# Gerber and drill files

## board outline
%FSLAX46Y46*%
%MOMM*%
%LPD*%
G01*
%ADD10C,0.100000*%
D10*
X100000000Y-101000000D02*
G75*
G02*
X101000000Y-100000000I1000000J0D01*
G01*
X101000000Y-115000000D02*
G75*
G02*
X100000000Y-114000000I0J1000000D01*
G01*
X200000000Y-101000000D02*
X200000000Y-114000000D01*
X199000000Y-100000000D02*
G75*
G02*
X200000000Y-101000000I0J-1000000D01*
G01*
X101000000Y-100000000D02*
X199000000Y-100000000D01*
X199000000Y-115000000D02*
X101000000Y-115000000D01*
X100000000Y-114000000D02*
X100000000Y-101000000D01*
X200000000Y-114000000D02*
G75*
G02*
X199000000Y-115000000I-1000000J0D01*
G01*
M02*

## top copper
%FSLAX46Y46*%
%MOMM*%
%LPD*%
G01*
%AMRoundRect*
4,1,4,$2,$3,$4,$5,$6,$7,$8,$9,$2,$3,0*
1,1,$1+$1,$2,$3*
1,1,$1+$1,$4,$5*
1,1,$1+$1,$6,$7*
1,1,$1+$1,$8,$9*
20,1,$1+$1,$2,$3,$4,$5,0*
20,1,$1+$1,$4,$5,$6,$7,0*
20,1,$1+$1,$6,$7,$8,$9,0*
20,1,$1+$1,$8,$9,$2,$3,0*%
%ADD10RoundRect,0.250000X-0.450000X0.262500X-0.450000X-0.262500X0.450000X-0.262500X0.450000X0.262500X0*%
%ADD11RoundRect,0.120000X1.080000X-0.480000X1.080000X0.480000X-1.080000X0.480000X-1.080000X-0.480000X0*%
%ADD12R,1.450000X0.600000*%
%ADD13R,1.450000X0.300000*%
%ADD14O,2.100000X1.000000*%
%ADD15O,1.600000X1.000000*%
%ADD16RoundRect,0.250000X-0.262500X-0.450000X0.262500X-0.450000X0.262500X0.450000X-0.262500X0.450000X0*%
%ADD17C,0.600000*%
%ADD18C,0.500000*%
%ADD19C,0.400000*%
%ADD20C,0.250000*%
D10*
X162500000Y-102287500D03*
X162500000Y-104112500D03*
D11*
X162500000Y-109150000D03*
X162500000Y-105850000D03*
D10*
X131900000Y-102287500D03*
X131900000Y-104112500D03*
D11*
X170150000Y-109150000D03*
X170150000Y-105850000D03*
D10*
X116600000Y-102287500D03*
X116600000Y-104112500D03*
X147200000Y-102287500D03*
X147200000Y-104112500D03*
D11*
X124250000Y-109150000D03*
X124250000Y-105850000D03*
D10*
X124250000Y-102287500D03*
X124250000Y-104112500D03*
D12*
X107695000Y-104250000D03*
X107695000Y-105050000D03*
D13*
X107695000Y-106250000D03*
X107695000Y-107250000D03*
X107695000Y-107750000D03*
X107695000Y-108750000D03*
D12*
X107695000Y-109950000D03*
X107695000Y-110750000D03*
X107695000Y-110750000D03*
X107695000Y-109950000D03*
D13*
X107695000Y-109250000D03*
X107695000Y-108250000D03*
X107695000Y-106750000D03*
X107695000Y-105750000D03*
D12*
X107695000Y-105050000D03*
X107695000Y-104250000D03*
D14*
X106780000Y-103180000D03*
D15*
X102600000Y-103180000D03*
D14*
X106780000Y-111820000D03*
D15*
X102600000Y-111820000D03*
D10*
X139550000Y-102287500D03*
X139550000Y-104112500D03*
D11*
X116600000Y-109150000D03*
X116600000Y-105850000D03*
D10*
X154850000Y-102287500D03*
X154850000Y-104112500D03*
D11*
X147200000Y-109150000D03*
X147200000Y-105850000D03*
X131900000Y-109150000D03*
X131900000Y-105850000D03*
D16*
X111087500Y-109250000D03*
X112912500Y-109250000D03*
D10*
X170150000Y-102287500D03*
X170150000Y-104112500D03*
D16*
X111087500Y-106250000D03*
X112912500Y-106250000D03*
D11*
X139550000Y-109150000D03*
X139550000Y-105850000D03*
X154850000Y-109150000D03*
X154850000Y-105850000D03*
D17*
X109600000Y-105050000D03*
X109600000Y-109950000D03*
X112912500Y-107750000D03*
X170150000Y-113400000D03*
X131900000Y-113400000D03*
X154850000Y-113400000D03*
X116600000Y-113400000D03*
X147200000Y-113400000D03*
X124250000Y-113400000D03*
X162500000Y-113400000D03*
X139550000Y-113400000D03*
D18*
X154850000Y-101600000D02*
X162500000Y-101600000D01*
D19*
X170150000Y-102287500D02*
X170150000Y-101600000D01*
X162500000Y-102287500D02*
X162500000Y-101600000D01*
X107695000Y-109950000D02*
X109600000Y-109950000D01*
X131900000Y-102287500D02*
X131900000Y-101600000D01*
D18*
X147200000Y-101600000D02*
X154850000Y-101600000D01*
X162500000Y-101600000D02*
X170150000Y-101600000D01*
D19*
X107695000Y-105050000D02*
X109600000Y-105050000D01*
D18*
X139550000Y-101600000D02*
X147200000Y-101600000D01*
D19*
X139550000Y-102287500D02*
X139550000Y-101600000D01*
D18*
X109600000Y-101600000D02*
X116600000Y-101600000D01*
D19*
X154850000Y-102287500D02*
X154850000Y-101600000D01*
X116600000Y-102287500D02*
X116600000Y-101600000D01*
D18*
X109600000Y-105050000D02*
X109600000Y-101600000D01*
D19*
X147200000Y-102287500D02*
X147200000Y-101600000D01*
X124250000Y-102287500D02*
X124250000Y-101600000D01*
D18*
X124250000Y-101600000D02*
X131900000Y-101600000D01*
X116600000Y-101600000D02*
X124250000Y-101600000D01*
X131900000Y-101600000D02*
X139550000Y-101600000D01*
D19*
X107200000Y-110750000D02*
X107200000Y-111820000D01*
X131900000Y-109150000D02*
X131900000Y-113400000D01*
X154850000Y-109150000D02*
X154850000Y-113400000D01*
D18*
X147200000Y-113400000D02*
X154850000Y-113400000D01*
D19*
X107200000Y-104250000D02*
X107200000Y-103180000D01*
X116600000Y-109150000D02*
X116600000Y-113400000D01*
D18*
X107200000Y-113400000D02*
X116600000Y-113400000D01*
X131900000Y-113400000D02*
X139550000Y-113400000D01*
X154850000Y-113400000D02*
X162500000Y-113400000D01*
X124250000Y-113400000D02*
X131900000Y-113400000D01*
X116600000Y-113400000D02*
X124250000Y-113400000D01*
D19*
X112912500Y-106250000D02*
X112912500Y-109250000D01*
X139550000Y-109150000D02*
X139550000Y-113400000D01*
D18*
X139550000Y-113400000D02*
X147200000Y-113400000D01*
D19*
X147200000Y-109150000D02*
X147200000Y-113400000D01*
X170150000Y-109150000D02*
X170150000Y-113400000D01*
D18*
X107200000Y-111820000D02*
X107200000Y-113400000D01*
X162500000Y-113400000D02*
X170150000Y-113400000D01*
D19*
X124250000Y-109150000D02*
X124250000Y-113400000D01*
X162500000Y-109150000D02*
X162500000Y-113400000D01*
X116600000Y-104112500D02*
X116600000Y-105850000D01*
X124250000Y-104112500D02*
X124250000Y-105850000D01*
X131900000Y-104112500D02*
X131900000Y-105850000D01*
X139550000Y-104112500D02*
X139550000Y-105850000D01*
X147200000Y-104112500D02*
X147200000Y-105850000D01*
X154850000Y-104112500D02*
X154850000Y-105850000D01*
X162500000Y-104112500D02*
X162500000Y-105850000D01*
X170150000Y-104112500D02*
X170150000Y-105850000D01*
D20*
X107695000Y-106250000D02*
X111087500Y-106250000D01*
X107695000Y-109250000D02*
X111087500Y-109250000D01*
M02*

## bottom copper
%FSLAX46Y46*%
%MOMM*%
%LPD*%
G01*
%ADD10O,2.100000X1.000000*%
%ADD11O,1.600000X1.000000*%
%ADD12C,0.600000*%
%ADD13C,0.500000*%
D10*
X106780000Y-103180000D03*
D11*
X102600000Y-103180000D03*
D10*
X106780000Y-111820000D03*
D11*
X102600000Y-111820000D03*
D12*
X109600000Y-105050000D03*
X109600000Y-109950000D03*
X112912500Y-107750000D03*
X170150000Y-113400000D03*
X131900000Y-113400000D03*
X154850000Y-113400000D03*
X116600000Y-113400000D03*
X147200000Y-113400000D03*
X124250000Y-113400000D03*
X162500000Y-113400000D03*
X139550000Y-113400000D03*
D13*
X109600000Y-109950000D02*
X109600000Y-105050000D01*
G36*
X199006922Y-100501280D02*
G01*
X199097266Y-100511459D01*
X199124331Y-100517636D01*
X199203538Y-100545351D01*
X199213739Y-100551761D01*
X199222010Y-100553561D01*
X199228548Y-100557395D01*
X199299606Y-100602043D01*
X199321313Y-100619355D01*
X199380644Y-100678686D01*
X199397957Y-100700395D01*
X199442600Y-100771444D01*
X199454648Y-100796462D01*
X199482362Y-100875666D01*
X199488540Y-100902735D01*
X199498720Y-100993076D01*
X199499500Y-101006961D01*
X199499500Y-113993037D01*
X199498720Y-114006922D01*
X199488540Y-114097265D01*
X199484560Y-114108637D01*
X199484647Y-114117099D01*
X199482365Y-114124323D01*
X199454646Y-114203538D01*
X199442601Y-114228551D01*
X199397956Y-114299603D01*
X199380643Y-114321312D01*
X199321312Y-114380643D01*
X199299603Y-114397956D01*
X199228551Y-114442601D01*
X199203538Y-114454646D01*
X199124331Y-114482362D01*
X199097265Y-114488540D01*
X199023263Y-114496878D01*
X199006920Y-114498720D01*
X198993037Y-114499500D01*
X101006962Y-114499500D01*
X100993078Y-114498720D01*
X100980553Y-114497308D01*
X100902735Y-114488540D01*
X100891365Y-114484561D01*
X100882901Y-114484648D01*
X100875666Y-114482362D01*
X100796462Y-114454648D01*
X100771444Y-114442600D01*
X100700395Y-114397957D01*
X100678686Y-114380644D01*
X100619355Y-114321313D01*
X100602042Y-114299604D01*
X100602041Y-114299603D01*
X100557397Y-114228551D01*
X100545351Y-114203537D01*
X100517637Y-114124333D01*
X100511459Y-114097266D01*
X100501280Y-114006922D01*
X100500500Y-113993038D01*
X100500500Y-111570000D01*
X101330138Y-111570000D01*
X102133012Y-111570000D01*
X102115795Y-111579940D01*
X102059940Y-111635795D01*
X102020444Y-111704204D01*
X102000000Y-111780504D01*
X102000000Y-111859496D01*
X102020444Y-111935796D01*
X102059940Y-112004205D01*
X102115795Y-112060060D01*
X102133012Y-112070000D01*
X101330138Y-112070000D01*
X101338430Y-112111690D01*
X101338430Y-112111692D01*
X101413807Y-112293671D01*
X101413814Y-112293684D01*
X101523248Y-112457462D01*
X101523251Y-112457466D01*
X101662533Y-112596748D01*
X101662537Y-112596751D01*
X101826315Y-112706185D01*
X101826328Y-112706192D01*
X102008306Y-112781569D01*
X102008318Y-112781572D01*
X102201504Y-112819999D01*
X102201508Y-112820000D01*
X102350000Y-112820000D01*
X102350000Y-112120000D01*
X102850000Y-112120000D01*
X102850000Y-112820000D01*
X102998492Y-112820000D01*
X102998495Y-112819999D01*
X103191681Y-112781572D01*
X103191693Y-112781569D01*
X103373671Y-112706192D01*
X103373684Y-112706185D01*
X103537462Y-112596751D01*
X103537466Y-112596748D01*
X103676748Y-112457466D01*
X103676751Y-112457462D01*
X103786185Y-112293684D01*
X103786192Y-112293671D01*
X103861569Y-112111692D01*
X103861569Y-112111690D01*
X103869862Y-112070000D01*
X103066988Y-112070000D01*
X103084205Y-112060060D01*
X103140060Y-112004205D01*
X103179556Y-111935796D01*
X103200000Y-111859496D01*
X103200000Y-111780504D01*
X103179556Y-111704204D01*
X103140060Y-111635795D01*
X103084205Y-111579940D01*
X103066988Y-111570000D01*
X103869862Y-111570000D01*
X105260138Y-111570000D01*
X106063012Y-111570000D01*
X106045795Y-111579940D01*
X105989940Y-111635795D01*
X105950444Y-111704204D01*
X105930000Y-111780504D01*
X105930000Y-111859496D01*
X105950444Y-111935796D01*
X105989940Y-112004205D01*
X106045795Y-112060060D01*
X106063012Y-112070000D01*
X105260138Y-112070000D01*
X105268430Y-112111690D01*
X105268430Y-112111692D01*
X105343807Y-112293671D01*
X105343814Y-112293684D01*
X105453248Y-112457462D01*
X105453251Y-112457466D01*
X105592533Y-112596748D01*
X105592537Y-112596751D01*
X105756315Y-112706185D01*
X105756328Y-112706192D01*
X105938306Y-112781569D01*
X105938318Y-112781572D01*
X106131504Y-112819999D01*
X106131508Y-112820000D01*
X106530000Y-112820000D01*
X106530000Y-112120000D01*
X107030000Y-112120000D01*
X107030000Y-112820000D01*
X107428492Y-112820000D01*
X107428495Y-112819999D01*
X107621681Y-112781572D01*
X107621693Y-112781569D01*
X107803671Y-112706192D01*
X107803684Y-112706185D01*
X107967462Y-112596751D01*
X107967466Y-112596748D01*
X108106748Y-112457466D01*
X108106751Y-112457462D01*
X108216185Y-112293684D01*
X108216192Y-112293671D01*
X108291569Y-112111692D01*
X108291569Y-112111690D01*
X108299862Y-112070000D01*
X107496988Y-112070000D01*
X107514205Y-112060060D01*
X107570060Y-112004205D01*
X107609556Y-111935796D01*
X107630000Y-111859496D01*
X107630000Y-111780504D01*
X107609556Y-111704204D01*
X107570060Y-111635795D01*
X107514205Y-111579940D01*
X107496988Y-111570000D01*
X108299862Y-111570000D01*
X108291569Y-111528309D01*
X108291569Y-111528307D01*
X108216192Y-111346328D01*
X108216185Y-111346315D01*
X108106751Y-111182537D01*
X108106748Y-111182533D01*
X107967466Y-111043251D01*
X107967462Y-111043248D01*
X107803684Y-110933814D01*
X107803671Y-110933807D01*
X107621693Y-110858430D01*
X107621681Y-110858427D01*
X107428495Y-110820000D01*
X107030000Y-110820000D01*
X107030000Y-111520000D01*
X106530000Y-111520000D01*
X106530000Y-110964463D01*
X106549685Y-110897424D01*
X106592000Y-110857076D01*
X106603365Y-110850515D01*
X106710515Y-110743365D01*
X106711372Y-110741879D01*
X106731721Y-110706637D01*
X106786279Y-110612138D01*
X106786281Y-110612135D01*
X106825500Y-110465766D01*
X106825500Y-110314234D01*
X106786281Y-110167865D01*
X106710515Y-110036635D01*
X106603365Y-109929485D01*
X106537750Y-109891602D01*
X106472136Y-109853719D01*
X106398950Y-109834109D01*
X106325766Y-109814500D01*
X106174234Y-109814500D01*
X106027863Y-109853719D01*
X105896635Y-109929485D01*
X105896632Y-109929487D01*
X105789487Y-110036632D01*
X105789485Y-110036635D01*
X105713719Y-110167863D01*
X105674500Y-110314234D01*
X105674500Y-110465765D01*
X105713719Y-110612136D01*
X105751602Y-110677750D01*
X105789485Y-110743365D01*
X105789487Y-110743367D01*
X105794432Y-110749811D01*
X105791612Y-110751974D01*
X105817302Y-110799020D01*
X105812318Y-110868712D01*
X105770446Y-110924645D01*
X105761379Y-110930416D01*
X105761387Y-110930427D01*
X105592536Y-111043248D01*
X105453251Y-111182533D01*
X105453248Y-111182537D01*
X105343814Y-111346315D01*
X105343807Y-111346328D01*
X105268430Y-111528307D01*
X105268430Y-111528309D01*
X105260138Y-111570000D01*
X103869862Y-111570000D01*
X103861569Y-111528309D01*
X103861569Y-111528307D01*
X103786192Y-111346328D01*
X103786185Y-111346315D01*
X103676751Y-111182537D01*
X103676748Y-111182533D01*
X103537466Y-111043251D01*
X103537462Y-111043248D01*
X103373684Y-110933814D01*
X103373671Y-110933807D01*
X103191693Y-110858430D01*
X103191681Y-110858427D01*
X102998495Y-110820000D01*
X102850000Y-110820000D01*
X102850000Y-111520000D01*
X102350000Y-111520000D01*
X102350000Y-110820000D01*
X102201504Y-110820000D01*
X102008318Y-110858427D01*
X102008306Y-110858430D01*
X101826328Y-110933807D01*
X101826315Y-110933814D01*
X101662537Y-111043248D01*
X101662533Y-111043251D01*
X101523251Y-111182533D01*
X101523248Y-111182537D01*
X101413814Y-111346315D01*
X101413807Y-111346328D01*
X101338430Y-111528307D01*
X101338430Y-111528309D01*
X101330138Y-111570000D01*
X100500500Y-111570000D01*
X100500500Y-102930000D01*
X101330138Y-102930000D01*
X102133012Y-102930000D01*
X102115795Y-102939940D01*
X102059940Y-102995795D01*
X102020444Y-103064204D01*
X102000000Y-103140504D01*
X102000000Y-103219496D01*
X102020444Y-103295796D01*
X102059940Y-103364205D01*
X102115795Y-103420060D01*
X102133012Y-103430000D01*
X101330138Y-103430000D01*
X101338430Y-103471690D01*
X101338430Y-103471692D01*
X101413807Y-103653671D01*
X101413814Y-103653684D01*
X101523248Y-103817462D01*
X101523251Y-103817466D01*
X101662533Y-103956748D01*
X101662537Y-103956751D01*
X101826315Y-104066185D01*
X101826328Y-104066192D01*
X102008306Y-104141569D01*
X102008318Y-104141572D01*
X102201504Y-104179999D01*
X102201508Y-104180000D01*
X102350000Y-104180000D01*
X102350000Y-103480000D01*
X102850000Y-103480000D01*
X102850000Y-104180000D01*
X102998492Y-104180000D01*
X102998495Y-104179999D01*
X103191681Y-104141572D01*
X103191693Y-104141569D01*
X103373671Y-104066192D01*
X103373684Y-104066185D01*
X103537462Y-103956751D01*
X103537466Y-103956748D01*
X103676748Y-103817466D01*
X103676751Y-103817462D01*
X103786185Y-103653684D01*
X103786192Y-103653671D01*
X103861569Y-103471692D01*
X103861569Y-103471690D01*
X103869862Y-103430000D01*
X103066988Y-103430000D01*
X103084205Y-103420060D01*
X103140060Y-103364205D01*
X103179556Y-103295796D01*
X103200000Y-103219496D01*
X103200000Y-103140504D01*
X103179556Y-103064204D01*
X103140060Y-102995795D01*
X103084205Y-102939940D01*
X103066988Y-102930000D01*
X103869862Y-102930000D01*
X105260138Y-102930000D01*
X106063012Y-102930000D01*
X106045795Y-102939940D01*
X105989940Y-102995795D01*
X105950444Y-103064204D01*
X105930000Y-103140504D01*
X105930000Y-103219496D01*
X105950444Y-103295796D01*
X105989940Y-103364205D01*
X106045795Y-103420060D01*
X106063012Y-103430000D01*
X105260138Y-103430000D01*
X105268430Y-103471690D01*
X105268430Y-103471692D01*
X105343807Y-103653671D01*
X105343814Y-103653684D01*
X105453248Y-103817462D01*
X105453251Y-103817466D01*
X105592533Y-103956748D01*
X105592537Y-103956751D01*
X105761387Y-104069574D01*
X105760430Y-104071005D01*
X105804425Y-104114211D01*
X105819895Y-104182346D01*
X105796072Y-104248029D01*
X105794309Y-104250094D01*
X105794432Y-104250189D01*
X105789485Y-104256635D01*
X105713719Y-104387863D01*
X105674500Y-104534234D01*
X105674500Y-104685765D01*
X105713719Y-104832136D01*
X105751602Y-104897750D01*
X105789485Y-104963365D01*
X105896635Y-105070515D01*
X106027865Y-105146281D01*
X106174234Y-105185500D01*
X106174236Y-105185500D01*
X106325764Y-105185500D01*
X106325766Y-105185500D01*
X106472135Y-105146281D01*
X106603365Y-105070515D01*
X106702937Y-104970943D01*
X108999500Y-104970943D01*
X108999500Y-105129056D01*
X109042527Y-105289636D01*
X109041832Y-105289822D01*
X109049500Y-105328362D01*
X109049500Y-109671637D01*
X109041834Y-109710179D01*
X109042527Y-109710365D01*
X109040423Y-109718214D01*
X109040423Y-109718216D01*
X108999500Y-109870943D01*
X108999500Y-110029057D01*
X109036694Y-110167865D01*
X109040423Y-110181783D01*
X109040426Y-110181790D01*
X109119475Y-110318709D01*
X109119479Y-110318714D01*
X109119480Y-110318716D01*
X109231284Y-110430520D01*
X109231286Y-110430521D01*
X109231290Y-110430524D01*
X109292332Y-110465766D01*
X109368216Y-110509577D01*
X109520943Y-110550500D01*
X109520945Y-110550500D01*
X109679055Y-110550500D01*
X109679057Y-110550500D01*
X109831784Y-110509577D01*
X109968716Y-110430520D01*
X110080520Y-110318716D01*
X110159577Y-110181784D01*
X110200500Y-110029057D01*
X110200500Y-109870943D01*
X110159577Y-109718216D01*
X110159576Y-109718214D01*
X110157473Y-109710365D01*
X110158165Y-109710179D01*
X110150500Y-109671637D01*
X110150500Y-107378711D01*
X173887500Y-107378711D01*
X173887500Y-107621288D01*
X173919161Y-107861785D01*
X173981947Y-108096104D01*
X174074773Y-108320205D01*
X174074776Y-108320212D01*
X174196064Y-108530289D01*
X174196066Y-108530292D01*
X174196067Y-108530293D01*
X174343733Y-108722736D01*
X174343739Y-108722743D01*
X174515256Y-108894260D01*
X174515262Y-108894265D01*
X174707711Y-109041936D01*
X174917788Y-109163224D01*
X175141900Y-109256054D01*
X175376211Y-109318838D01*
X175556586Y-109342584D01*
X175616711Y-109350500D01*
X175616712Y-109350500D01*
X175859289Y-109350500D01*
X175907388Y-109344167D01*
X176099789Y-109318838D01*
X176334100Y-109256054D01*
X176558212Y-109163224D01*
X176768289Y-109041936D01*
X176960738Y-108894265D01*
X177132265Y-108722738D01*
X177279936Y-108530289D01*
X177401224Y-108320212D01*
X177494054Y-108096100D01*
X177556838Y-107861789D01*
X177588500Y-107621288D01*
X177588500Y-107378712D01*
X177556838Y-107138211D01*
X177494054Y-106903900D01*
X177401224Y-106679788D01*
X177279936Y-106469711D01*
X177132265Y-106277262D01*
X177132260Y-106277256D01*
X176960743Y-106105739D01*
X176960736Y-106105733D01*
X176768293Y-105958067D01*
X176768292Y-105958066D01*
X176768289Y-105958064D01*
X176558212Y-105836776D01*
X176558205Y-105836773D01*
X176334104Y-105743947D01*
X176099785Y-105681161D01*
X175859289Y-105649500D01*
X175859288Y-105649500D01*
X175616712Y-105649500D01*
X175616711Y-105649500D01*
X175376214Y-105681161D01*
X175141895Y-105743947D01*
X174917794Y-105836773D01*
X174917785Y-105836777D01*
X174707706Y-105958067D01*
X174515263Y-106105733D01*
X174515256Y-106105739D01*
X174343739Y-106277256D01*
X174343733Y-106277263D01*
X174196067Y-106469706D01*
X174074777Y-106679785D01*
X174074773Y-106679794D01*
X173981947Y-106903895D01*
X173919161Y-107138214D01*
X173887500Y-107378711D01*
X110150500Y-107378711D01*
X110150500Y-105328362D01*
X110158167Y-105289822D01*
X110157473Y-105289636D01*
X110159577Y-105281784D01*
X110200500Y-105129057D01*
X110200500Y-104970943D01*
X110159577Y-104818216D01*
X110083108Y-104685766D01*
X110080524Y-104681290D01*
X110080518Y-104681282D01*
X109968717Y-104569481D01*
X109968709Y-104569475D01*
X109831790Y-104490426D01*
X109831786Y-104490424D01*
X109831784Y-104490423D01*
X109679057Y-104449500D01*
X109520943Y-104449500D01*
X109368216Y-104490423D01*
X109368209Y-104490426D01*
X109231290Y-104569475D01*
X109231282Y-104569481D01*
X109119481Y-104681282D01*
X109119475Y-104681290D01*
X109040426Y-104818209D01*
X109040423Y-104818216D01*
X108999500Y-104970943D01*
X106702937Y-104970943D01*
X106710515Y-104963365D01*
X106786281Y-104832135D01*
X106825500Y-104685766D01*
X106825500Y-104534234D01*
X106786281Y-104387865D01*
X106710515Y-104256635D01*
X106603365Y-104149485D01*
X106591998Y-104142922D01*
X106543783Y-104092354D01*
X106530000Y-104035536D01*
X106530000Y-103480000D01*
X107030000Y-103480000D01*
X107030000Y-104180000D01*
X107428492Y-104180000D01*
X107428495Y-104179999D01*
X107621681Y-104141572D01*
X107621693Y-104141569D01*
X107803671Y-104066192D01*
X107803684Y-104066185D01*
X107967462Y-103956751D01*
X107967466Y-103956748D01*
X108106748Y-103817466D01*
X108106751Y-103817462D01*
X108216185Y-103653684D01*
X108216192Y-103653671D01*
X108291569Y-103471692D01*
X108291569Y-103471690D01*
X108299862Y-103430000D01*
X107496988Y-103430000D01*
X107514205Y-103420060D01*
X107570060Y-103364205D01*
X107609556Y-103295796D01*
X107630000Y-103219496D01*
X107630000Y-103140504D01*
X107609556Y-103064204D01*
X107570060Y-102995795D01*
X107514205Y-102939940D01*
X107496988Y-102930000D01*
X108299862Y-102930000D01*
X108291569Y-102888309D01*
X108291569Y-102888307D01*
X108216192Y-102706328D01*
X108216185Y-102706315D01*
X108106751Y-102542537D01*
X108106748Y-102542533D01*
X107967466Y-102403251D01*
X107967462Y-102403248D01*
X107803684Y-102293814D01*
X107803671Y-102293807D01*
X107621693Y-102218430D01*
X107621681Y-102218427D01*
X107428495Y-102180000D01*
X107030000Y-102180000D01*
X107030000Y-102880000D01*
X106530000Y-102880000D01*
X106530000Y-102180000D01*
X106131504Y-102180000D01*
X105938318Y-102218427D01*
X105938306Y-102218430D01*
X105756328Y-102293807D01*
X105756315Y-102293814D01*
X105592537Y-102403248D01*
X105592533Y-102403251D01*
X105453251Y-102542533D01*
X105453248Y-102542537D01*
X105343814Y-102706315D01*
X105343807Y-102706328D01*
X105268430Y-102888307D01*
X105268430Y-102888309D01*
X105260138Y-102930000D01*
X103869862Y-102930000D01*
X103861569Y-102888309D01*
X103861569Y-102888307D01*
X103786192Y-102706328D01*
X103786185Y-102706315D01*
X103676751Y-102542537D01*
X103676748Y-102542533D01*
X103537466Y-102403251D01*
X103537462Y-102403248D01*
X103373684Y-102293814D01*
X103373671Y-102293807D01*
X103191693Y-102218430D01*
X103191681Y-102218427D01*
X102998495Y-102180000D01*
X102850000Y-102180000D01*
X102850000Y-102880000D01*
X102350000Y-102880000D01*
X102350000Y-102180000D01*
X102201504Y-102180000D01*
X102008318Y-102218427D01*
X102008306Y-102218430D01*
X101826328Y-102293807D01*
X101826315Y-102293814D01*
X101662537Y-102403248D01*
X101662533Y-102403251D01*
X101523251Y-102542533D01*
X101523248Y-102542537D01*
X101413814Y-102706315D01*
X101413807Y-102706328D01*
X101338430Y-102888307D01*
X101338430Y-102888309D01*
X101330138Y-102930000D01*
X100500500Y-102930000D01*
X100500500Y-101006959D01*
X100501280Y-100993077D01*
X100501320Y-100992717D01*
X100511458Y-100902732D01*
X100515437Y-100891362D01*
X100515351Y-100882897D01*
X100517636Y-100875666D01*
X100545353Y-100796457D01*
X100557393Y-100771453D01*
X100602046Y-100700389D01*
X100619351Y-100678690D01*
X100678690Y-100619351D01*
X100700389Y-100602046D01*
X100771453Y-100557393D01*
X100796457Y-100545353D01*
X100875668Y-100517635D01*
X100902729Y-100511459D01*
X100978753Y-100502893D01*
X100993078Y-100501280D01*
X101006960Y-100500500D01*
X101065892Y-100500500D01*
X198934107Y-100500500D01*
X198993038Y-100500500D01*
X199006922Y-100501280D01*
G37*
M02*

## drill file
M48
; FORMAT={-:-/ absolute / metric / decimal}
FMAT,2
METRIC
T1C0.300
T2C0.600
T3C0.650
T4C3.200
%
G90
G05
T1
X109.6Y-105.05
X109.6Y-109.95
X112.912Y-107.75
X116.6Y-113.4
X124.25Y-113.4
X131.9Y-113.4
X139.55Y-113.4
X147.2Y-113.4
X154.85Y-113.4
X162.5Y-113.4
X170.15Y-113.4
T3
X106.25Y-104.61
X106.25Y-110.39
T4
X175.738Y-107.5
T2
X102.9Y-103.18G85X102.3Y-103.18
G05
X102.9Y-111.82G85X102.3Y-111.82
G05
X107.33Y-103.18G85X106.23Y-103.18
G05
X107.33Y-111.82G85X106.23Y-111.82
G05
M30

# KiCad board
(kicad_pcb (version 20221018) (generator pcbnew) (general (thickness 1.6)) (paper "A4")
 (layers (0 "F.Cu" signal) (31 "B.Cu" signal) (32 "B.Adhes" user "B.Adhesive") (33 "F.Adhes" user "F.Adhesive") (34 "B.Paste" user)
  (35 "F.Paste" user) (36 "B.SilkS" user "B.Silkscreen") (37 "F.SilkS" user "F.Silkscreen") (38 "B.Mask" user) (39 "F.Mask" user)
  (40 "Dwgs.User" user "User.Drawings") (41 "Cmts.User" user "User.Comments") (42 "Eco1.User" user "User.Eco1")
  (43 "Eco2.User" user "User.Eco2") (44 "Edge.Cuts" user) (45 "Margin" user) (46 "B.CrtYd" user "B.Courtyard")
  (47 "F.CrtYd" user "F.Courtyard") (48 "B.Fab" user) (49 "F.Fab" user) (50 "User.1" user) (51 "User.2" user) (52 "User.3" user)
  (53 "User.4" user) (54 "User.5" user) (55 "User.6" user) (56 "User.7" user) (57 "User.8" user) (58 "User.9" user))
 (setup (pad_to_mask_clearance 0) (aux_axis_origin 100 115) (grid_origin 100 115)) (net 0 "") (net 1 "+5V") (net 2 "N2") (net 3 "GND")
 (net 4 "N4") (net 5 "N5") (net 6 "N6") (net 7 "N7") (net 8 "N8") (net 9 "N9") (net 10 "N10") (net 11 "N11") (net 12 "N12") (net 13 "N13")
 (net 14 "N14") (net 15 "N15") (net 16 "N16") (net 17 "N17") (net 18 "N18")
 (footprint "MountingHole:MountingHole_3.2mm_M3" (layer "F.Cu") (at 175.738 107.5)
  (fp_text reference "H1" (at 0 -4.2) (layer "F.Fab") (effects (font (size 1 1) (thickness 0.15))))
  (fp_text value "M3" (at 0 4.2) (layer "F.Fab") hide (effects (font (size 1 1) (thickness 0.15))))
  (pad "" np_thru_hole circle (at 0 0) (size 3.2 3.2) (drill 3.2) (layers "*.Cu" "*.Mask")))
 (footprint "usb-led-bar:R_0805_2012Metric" (layer "F.Cu") (at 162.5 103.2 -90)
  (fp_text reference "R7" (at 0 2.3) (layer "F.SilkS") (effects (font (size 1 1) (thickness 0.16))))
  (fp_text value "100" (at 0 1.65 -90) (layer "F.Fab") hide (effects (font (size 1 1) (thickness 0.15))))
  (pad "1" smd roundrect (at -0.9125 0 270) (size 1.025 1.4) (layers "F.Cu" "F.Paste" "F.Mask") (roundrect_rratio 0.243902) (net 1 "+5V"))
  (pad "2" smd roundrect (at 0.9125 0 270) (size 1.025 1.4) (layers "F.Cu" "F.Paste" "F.Mask") (roundrect_rratio 0.243902) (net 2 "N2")))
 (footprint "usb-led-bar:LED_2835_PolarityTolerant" (layer "F.Cu") (at 162.5 107.5 90)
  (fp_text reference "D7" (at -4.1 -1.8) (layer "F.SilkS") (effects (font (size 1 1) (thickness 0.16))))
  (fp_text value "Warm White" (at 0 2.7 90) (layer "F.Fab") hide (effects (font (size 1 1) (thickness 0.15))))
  (pad "1" smd roundrect (at -1.65 0 90) (size 1.2 2.4) (layers "F.Cu" "F.Paste" "F.Mask") (roundrect_rratio 0.1) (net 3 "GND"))
  (pad "2" smd roundrect (at 1.65 0 90) (size 1.2 2.4) (layers "F.Cu" "F.Paste" "F.Mask") (roundrect_rratio 0.1) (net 2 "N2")))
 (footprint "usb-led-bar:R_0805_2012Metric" (layer "F.Cu") (at 131.9 103.2 -90)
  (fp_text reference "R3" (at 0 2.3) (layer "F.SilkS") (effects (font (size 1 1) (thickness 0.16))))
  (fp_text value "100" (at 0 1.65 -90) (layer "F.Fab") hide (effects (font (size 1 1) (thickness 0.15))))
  (pad "1" smd roundrect (at -0.9125 0 270) (size 1.025 1.4) (layers "F.Cu" "F.Paste" "F.Mask") (roundrect_rratio 0.243902) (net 1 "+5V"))
  (pad "2" smd roundrect (at 0.9125 0 270) (size 1.025 1.4) (layers "F.Cu" "F.Paste" "F.Mask") (roundrect_rratio 0.243902) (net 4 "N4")))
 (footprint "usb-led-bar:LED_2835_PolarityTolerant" (layer "F.Cu") (at 170.15 107.5 90)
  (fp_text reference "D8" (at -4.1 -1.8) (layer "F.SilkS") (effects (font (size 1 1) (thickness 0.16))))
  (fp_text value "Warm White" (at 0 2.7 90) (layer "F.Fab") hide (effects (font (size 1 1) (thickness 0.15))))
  (pad "1" smd roundrect (at -1.65 0 90) (size 1.2 2.4) (layers "F.Cu" "F.Paste" "F.Mask") (roundrect_rratio 0.1) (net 3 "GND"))
  (pad "2" smd roundrect (at 1.65 0 90) (size 1.2 2.4) (layers "F.Cu" "F.Paste" "F.Mask") (roundrect_rratio 0.1) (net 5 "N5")))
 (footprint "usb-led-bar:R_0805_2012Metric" (layer "F.Cu") (at 116.6 103.2 -90)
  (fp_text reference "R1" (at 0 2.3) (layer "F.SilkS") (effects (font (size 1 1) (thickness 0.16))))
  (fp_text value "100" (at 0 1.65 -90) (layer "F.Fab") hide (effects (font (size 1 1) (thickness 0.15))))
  (pad "1" smd roundrect (at -0.9125 0 270) (size 1.025 1.4) (layers "F.Cu" "F.Paste" "F.Mask") (roundrect_rratio 0.243902) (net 1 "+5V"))
  (pad "2" smd roundrect (at 0.9125 0 270) (size 1.025 1.4) (layers "F.Cu" "F.Paste" "F.Mask") (roundrect_rratio 0.243902) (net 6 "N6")))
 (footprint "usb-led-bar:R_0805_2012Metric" (layer "F.Cu") (at 147.2 103.2 -90)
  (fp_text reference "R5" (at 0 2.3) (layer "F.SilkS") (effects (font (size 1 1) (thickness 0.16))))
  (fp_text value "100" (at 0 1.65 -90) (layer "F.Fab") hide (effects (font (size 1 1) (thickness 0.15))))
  (pad "1" smd roundrect (at -0.9125 0 270) (size 1.025 1.4) (layers "F.Cu" "F.Paste" "F.Mask") (roundrect_rratio 0.243902) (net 1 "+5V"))
  (pad "2" smd roundrect (at 0.9125 0 270) (size 1.025 1.4) (layers "F.Cu" "F.Paste" "F.Mask") (roundrect_rratio 0.243902) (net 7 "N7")))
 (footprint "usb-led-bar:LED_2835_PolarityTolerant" (layer "F.Cu") (at 124.25 107.5 90)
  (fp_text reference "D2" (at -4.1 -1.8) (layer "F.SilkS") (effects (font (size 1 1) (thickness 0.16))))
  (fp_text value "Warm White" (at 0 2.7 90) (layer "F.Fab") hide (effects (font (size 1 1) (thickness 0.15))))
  (pad "1" smd roundrect (at -1.65 0 90) (size 1.2 2.4) (layers "F.Cu" "F.Paste" "F.Mask") (roundrect_rratio 0.1) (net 3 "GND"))
  (pad "2" smd roundrect (at 1.65 0 90) (size 1.2 2.4) (layers "F.Cu" "F.Paste" "F.Mask") (roundrect_rratio 0.1) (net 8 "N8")))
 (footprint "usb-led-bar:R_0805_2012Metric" (layer "F.Cu") (at 124.25 103.2 -90)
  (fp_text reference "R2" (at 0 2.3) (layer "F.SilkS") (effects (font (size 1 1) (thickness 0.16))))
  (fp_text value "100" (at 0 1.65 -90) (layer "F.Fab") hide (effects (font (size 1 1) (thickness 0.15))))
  (pad "1" smd roundrect (at -0.9125 0 270) (size 1.025 1.4) (layers "F.Cu" "F.Paste" "F.Mask") (roundrect_rratio 0.243902) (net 1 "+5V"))
  (pad "2" smd roundrect (at 0.9125 0 270) (size 1.025 1.4) (layers "F.Cu" "F.Paste" "F.Mask") (roundrect_rratio 0.243902) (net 8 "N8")))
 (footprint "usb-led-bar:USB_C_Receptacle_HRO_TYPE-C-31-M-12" (layer "F.Cu") (at 103.65 107.5 -90)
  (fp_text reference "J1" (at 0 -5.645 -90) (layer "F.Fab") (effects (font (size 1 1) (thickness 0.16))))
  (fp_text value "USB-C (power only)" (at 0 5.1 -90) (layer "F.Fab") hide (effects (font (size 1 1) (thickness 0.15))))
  (pad "" np_thru_hole circle (at -2.89 -2.6 270) (size 0.65 0.65) (drill 0.65) (layers "*.Cu" "*.Mask"))
  (pad "" np_thru_hole circle (at 2.89 -2.6 270) (size 0.65 0.65) (drill 0.65) (layers "*.Cu" "*.Mask"))
  (pad "A1" smd rect (at -3.25 -4.045 270) (size 0.6 1.45) (layers "F.Cu" "F.Paste" "F.Mask") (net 3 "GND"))
  (pad "A4" smd rect (at -2.45 -4.045 270) (size 0.6 1.45) (layers "F.Cu" "F.Paste" "F.Mask") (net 1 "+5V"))
  (pad "A5" smd rect (at -1.25 -4.045 270) (size 0.3 1.45) (layers "F.Cu" "F.Paste" "F.Mask") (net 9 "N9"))
  (pad "A6" smd rect (at -0.25 -4.045 270) (size 0.3 1.45) (layers "F.Cu" "F.Paste" "F.Mask") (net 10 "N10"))
  (pad "A7" smd rect (at 0.25 -4.045 270) (size 0.3 1.45) (layers "F.Cu" "F.Paste" "F.Mask") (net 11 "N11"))
  (pad "A8" smd rect (at 1.25 -4.045 270) (size 0.3 1.45) (layers "F.Cu" "F.Paste" "F.Mask") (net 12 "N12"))
  (pad "A9" smd rect (at 2.45 -4.045 270) (size 0.6 1.45) (layers "F.Cu" "F.Paste" "F.Mask") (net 1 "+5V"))
  (pad "A12" smd rect (at 3.25 -4.045 270) (size 0.6 1.45) (layers "F.Cu" "F.Paste" "F.Mask") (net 3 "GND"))
  (pad "B1" smd rect (at 3.25 -4.045 270) (size 0.6 1.45) (layers "F.Cu" "F.Paste" "F.Mask") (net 3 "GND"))
  (pad "B4" smd rect (at 2.45 -4.045 270) (size 0.6 1.45) (layers "F.Cu" "F.Paste" "F.Mask") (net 1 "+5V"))
  (pad "B5" smd rect (at 1.75 -4.045 270) (size 0.3 1.45) (layers "F.Cu" "F.Paste" "F.Mask") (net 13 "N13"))
  (pad "B6" smd rect (at 0.75 -4.045 270) (size 0.3 1.45) (layers "F.Cu" "F.Paste" "F.Mask") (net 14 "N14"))
  (pad "B7" smd rect (at -0.75 -4.045 270) (size 0.3 1.45) (layers "F.Cu" "F.Paste" "F.Mask") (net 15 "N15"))
  (pad "B8" smd rect (at -1.75 -4.045 270) (size 0.3 1.45) (layers "F.Cu" "F.Paste" "F.Mask") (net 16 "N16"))
  (pad "B9" smd rect (at -2.45 -4.045 270) (size 0.6 1.45) (layers "F.Cu" "F.Paste" "F.Mask") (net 1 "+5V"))
  (pad "B12" smd rect (at -3.25 -4.045 270) (size 0.6 1.45) (layers "F.Cu" "F.Paste" "F.Mask") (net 3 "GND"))
  (pad "S1" thru_hole oval (at -4.32 -3.13 270) (size 1 2.1) (drill oval 0.6 1.7) (layers "*.Cu" "*.Mask") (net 3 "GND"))
  (pad "S1" thru_hole oval (at -4.32 1.05 270) (size 1 1.6) (drill oval 0.6 1.2) (layers "*.Cu" "*.Mask") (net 3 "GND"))
  (pad "S1" thru_hole oval (at 4.32 -3.13 270) (size 1 2.1) (drill oval 0.6 1.7) (layers "*.Cu" "*.Mask") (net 3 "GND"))
  (pad "S1" thru_hole oval (at 4.32 1.05 270) (size 1 1.6) (drill oval 0.6 1.2) (layers "*.Cu" "*.Mask") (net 3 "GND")))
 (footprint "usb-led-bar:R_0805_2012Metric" (layer "F.Cu") (at 139.55 103.2 -90)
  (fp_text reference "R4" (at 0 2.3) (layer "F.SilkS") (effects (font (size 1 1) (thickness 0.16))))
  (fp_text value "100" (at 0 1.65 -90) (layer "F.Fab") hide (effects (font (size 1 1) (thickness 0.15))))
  (pad "1" smd roundrect (at -0.9125 0 270) (size 1.025 1.4) (layers "F.Cu" "F.Paste" "F.Mask") (roundrect_rratio 0.243902) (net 1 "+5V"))
  (pad "2" smd roundrect (at 0.9125 0 270) (size 1.025 1.4) (layers "F.Cu" "F.Paste" "F.Mask") (roundrect_rratio 0.243902) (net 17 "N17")))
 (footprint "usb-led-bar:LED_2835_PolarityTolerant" (layer "F.Cu") (at 116.6 107.5 90)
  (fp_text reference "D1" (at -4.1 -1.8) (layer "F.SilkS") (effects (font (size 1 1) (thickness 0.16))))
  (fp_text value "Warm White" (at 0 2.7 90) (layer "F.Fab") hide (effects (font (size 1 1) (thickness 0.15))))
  (pad "1" smd roundrect (at -1.65 0 90) (size 1.2 2.4) (layers "F.Cu" "F.Paste" "F.Mask") (roundrect_rratio 0.1) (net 3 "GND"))
  (pad "2" smd roundrect (at 1.65 0 90) (size 1.2 2.4) (layers "F.Cu" "F.Paste" "F.Mask") (roundrect_rratio 0.1) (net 6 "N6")))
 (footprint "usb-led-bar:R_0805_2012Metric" (layer "F.Cu") (at 154.85 103.2 -90)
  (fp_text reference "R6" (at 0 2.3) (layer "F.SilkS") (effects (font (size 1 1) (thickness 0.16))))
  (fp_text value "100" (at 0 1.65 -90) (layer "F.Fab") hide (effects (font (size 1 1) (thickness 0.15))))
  (pad "1" smd roundrect (at -0.9125 0 270) (size 1.025 1.4) (layers "F.Cu" "F.Paste" "F.Mask") (roundrect_rratio 0.243902) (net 1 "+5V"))
  (pad "2" smd roundrect (at 0.9125 0 270) (size 1.025 1.4) (layers "F.Cu" "F.Paste" "F.Mask") (roundrect_rratio 0.243902) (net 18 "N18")))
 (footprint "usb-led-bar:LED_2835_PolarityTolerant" (layer "F.Cu") (at 147.2 107.5 90)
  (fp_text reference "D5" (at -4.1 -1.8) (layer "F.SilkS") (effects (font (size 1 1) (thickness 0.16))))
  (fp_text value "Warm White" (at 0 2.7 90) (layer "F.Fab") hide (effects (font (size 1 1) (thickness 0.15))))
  (pad "1" smd roundrect (at -1.65 0 90) (size 1.2 2.4) (layers "F.Cu" "F.Paste" "F.Mask") (roundrect_rratio 0.1) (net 3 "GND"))
  (pad "2" smd roundrect (at 1.65 0 90) (size 1.2 2.4) (layers "F.Cu" "F.Paste" "F.Mask") (roundrect_rratio 0.1) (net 7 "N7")))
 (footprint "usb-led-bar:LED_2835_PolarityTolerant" (layer "F.Cu") (at 131.9 107.5 90)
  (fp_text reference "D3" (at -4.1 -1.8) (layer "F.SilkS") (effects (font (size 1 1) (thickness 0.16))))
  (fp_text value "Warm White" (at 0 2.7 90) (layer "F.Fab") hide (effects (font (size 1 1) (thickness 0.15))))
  (pad "1" smd roundrect (at -1.65 0 90) (size 1.2 2.4) (layers "F.Cu" "F.Paste" "F.Mask") (roundrect_rratio 0.1) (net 3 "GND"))
  (pad "2" smd roundrect (at 1.65 0 90) (size 1.2 2.4) (layers "F.Cu" "F.Paste" "F.Mask") (roundrect_rratio 0.1) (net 4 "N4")))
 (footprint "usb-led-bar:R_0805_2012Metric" (layer "F.Cu") (at 112 109.25)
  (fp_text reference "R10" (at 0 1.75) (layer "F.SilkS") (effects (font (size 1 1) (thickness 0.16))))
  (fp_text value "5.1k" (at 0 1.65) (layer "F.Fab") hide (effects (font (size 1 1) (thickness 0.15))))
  (pad "1" smd roundrect (at -0.9125 0) (size 1.025 1.4) (layers "F.Cu" "F.Paste" "F.Mask") (roundrect_rratio 0.243902) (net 13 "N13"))
  (pad "2" smd roundrect (at 0.9125 0) (size 1.025 1.4) (layers "F.Cu" "F.Paste" "F.Mask") (roundrect_rratio 0.243902) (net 3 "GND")))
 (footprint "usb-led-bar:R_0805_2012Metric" (layer "F.Cu") (at 170.15 103.2 -90)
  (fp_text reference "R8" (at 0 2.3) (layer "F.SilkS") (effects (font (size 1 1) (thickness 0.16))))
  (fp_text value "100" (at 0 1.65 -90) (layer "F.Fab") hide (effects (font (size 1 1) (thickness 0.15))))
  (pad "1" smd roundrect (at -0.9125 0 270) (size 1.025 1.4) (layers "F.Cu" "F.Paste" "F.Mask") (roundrect_rratio 0.243902) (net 1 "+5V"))
  (pad "2" smd roundrect (at 0.9125 0 270) (size 1.025 1.4) (layers "F.Cu" "F.Paste" "F.Mask") (roundrect_rratio 0.243902) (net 5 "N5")))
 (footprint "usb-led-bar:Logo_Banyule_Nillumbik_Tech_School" (layer "F.Cu") (at 189.244 107.5)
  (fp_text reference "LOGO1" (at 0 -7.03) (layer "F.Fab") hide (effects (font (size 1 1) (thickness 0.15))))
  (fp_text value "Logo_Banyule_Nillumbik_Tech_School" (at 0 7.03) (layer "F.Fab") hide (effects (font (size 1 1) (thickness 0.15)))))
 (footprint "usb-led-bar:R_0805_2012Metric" (layer "F.Cu") (at 112 106.25)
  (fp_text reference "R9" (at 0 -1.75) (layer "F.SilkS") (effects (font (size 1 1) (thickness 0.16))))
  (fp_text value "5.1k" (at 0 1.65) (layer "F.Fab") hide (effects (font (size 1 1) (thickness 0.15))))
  (pad "1" smd roundrect (at -0.9125 0) (size 1.025 1.4) (layers "F.Cu" "F.Paste" "F.Mask") (roundrect_rratio 0.243902) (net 9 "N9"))
  (pad "2" smd roundrect (at 0.9125 0) (size 1.025 1.4) (layers "F.Cu" "F.Paste" "F.Mask") (roundrect_rratio 0.243902) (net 3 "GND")))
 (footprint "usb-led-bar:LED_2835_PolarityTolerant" (layer "F.Cu") (at 139.55 107.5 90)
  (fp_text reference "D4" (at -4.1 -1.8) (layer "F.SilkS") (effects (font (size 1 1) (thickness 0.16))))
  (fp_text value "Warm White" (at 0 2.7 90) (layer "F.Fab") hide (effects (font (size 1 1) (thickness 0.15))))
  (pad "1" smd roundrect (at -1.65 0 90) (size 1.2 2.4) (layers "F.Cu" "F.Paste" "F.Mask") (roundrect_rratio 0.1) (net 3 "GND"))
  (pad "2" smd roundrect (at 1.65 0 90) (size 1.2 2.4) (layers "F.Cu" "F.Paste" "F.Mask") (roundrect_rratio 0.1) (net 17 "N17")))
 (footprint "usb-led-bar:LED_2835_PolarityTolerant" (layer "F.Cu") (at 154.85 107.5 90)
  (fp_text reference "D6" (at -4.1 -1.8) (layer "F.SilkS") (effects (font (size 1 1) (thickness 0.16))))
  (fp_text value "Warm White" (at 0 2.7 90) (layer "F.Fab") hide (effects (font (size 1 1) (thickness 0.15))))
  (pad "1" smd roundrect (at -1.65 0 90) (size 1.2 2.4) (layers "F.Cu" "F.Paste" "F.Mask") (roundrect_rratio 0.1) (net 3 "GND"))
  (pad "2" smd roundrect (at 1.65 0 90) (size 1.2 2.4) (layers "F.Cu" "F.Paste" "F.Mask") (roundrect_rratio 0.1) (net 18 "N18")))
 (gr_arc (start 100 101) (mid 100.292893 100.292893) (end 101 100) (stroke (width 0.1) (type default)) (layer "Edge.Cuts"))
 (gr_arc (start 101 115) (mid 100.292893 114.707106) (end 100 114) (stroke (width 0.1) (type default)) (layer "Edge.Cuts"))
 (gr_line (start 200 101) (end 200 114) (stroke (width 0.1) (type default)) (layer "Edge.Cuts"))
 (gr_arc (start 199 100) (mid 199.707106 100.292893) (end 200 101) (stroke (width 0.1) (type default)) (layer "Edge.Cuts"))
 (gr_line (start 101 100) (end 199 100) (stroke (width 0.1) (type default)) (layer "Edge.Cuts"))
 (gr_line (start 199 115) (end 101 115) (stroke (width 0.1) (type default)) (layer "Edge.Cuts"))
 (gr_line (start 100 114) (end 100 101) (stroke (width 0.1) (type default)) (layer "Edge.Cuts"))
 (gr_arc (start 200 114) (mid 199.707106 114.707106) (end 199 115) (stroke (width 0.1) (type default)) (layer "Edge.Cuts"))
 (segment (start 154.85 101.6) (end 162.5 101.6) (width 0.5) (layer "F.Cu") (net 1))
 (segment (start 170.15 102.2875) (end 170.15 101.6) (width 0.4) (layer "F.Cu") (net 1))
 (segment (start 162.5 102.2875) (end 162.5 101.6) (width 0.4) (layer "F.Cu") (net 1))
 (segment (start 107.695 109.95) (end 109.6 109.95) (width 0.4) (layer "F.Cu") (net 1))
 (segment (start 131.9 102.2875) (end 131.9 101.6) (width 0.4) (layer "F.Cu") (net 1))
 (segment (start 147.2 101.6) (end 154.85 101.6) (width 0.5) (layer "F.Cu") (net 1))
 (segment (start 162.5 101.6) (end 170.15 101.6) (width 0.5) (layer "F.Cu") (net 1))
 (segment (start 107.695 105.05) (end 109.6 105.05) (width 0.4) (layer "F.Cu") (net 1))
 (segment (start 139.55 101.6) (end 147.2 101.6) (width 0.5) (layer "F.Cu") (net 1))
 (segment (start 139.55 102.2875) (end 139.55 101.6) (width 0.4) (layer "F.Cu") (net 1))
 (segment (start 109.6 101.6) (end 116.6 101.6) (width 0.5) (layer "F.Cu") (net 1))
 (segment (start 154.85 102.2875) (end 154.85 101.6) (width 0.4) (layer "F.Cu") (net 1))
 (segment (start 116.6 102.2875) (end 116.6 101.6) (width 0.4) (layer "F.Cu") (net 1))
 (segment (start 109.6 105.05) (end 109.6 101.6) (width 0.5) (layer "F.Cu") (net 1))
 (segment (start 147.2 102.2875) (end 147.2 101.6) (width 0.4) (layer "F.Cu") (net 1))
 (segment (start 124.25 102.2875) (end 124.25 101.6) (width 0.4) (layer "F.Cu") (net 1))
 (segment (start 124.25 101.6) (end 131.9 101.6) (width 0.5) (layer "F.Cu") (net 1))
 (segment (start 116.6 101.6) (end 124.25 101.6) (width 0.5) (layer "F.Cu") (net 1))
 (segment (start 131.9 101.6) (end 139.55 101.6) (width 0.5) (layer "F.Cu") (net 1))
 (via (at 109.6 105.05) (size 0.6) (drill 0.3) (layers "F.Cu" "B.Cu") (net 1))
 (via (at 109.6 109.95) (size 0.6) (drill 0.3) (layers "F.Cu" "B.Cu") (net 1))
 (segment (start 109.6 109.95) (end 109.6 105.05) (width 0.5) (layer "B.Cu") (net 1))
 (segment (start 107.2 110.75) (end 107.2 111.82) (width 0.4) (layer "F.Cu") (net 3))
 (segment (start 131.9 109.15) (end 131.9 113.4) (width 0.4) (layer "F.Cu") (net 3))
 (segment (start 154.85 109.15) (end 154.85 113.4) (width 0.4) (layer "F.Cu") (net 3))
 (segment (start 147.2 113.4) (end 154.85 113.4) (width 0.5) (layer "F.Cu") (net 3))
 (segment (start 107.2 104.25) (end 107.2 103.18) (width 0.4) (layer "F.Cu") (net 3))
 (segment (start 116.6 109.15) (end 116.6 113.4) (width 0.4) (layer "F.Cu") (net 3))
 (segment (start 107.2 113.4) (end 116.6 113.4) (width 0.5) (layer "F.Cu") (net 3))
 (segment (start 131.9 113.4) (end 139.55 113.4) (width 0.5) (layer "F.Cu") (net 3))
 (segment (start 154.85 113.4) (end 162.5 113.4) (width 0.5) (layer "F.Cu") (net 3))
 (segment (start 124.25 113.4) (end 131.9 113.4) (width 0.5) (layer "F.Cu") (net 3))
 (segment (start 116.6 113.4) (end 124.25 113.4) (width 0.5) (layer "F.Cu") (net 3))
 (segment (start 112.9125 106.25) (end 112.9125 109.25) (width 0.4) (layer "F.Cu") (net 3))
 (segment (start 139.55 109.15) (end 139.55 113.4) (width 0.4) (layer "F.Cu") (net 3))
 (segment (start 139.55 113.4) (end 147.2 113.4) (width 0.5) (layer "F.Cu") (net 3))
 (segment (start 147.2 109.15) (end 147.2 113.4) (width 0.4) (layer "F.Cu") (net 3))
 (segment (start 170.15 109.15) (end 170.15 113.4) (width 0.4) (layer "F.Cu") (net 3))
 (segment (start 107.2 111.82) (end 107.2 113.4) (width 0.5) (layer "F.Cu") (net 3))
 (segment (start 162.5 113.4) (end 170.15 113.4) (width 0.5) (layer "F.Cu") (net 3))
 (segment (start 124.25 109.15) (end 124.25 113.4) (width 0.4) (layer "F.Cu") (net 3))
 (segment (start 162.5 109.15) (end 162.5 113.4) (width 0.4) (layer "F.Cu") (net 3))
 (via (at 112.9125 107.75) (size 0.6) (drill 0.3) (layers "F.Cu" "B.Cu") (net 3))
 (via (at 170.15 113.4) (size 0.6) (drill 0.3) (layers "F.Cu" "B.Cu") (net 3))
 (via (at 131.9 113.4) (size 0.6) (drill 0.3) (layers "F.Cu" "B.Cu") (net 3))
 (via (at 154.85 113.4) (size 0.6) (drill 0.3) (layers "F.Cu" "B.Cu") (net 3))
 (via (at 116.6 113.4) (size 0.6) (drill 0.3) (layers "F.Cu" "B.Cu") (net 3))
 (via (at 147.2 113.4) (size 0.6) (drill 0.3) (layers "F.Cu" "B.Cu") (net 3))
 (via (at 124.25 113.4) (size 0.6) (drill 0.3) (layers "F.Cu" "B.Cu") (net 3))
 (via (at 162.5 113.4) (size 0.6) (drill 0.3) (layers "F.Cu" "B.Cu") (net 3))
 (via (at 139.55 113.4) (size 0.6) (drill 0.3) (layers "F.Cu" "B.Cu") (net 3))
 (segment (start 116.6 104.1125) (end 116.6 105.85) (width 0.4) (layer "F.Cu") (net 6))
 (segment (start 124.25 104.1125) (end 124.25 105.85) (width 0.4) (layer "F.Cu") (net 8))
 (segment (start 131.9 104.1125) (end 131.9 105.85) (width 0.4) (layer "F.Cu") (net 4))
 (segment (start 139.55 104.1125) (end 139.55 105.85) (width 0.4) (layer "F.Cu") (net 17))
 (segment (start 147.2 104.1125) (end 147.2 105.85) (width 0.4) (layer "F.Cu") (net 7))
 (segment (start 154.85 104.1125) (end 154.85 105.85) (width 0.4) (layer "F.Cu") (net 18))
 (segment (start 162.5 104.1125) (end 162.5 105.85) (width 0.4) (layer "F.Cu") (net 2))
 (segment (start 170.15 104.1125) (end 170.15 105.85) (width 0.4) (layer "F.Cu") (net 5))
 (segment (start 107.695 106.25) (end 111.0875 106.25) (width 0.25) (layer "F.Cu") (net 9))
 (segment (start 107.695 109.25) (end 111.0875 109.25) (width 0.25) (layer "F.Cu") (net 13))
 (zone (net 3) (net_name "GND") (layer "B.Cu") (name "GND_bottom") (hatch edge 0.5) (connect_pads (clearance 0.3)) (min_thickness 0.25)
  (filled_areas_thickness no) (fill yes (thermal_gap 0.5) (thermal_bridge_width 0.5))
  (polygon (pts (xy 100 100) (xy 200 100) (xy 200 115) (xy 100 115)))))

